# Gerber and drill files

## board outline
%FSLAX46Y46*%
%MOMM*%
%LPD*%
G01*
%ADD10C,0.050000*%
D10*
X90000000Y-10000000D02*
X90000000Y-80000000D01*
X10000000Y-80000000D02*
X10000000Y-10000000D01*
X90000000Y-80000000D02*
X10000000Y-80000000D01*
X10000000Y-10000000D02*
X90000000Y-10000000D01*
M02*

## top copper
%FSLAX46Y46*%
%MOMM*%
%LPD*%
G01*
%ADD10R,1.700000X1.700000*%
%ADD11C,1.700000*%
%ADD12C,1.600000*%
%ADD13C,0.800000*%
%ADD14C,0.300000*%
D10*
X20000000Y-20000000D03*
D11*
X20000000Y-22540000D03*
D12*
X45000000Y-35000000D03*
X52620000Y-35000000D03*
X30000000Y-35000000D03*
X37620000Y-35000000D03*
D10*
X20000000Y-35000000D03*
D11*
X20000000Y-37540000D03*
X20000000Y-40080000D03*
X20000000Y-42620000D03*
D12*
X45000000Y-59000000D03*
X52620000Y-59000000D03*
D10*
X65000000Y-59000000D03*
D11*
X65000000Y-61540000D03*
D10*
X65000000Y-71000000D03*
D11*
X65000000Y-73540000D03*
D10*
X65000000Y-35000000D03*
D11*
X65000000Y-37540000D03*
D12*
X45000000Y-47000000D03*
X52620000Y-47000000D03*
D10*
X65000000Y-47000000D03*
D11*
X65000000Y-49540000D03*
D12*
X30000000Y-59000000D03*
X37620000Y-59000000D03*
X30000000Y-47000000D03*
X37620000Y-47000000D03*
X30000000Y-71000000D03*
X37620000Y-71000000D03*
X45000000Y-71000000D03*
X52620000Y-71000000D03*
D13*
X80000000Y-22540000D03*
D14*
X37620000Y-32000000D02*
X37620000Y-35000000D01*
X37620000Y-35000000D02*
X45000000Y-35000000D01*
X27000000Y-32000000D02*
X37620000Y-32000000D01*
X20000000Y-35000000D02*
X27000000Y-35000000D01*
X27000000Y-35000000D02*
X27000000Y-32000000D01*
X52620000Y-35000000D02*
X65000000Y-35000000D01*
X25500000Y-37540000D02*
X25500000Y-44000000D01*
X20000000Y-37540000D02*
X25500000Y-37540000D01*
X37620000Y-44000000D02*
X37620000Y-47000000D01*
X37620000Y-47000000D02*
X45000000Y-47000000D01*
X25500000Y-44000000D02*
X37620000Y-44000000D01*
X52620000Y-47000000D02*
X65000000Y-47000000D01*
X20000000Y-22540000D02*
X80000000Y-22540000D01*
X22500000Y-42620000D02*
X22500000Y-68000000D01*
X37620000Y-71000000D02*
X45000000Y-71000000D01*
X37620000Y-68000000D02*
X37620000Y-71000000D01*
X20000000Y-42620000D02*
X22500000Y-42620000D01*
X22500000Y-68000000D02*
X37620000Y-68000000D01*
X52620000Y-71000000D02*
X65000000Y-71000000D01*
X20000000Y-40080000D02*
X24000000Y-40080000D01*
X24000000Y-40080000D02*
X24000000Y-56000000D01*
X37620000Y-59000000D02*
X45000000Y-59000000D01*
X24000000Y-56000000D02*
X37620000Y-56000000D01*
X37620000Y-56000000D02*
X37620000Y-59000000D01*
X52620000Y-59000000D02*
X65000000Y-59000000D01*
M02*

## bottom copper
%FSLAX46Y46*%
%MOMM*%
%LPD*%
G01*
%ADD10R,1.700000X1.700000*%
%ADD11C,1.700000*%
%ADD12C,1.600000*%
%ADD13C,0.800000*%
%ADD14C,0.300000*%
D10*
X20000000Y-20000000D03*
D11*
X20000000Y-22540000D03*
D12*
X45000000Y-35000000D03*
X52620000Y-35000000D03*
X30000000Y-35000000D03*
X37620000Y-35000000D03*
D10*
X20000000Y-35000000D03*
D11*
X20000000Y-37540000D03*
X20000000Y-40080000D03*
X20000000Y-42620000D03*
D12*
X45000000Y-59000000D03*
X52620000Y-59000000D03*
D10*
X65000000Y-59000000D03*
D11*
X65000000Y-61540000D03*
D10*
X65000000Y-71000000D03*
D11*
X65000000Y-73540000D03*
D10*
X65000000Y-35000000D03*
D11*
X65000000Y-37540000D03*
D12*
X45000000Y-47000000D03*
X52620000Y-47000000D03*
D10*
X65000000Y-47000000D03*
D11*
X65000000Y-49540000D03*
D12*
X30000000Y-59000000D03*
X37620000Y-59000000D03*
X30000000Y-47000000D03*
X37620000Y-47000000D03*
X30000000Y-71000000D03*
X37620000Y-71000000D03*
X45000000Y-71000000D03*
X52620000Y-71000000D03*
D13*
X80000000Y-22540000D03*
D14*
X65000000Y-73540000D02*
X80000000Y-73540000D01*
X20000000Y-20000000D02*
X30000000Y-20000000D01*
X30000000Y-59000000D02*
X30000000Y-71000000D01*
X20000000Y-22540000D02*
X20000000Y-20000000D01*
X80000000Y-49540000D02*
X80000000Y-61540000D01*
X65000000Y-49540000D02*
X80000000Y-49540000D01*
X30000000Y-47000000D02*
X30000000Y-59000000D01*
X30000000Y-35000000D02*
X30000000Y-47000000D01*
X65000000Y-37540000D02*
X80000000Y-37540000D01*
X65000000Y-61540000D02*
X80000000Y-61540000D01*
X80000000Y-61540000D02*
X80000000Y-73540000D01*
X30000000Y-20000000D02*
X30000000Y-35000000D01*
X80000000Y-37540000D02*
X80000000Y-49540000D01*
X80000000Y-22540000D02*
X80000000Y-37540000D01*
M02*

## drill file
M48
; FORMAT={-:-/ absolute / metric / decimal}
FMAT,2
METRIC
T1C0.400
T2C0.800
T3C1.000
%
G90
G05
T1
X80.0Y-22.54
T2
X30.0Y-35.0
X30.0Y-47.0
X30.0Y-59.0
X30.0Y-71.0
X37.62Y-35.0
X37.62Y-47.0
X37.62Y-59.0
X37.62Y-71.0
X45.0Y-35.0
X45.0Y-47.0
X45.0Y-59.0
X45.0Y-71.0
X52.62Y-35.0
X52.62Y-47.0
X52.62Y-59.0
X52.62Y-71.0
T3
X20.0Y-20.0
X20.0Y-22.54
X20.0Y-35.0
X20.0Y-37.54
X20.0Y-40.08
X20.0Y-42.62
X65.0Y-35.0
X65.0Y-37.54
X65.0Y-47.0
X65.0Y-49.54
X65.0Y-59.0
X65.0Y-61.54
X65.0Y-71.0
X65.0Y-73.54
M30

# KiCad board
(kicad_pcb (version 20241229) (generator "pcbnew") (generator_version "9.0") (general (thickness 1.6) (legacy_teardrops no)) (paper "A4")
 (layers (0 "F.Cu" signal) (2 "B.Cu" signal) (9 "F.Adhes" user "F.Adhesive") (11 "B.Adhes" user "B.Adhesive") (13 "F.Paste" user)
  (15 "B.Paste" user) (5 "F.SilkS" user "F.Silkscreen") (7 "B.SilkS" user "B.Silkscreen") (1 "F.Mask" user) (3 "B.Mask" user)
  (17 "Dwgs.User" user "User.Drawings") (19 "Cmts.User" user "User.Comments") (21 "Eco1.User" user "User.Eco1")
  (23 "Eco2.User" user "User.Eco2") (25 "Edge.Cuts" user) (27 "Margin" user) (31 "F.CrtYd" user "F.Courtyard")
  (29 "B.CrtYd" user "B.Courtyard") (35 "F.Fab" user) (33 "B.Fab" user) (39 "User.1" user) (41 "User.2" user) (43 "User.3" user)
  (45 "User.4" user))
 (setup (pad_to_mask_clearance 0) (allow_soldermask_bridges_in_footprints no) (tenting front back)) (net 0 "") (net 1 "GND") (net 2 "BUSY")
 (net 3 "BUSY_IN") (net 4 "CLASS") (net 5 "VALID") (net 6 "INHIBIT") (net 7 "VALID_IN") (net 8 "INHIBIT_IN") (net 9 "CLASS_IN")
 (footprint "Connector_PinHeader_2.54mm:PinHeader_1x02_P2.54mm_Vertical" (layer "F.Cu") (at 20 20)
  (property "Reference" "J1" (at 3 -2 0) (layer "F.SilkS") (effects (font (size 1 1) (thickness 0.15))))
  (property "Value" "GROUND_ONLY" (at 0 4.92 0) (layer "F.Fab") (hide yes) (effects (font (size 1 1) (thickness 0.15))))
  (pad "1" thru_hole rect (at 0 0) (size 1.7 1.7) (drill 1) (layers "*.Cu" "*.Mask") (remove_unused_layers no) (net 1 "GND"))
  (pad "2" thru_hole circle (at 0 2.54) (size 1.7 1.7) (drill 1) (layers "*.Cu" "*.Mask") (remove_unused_layers no) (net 1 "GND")))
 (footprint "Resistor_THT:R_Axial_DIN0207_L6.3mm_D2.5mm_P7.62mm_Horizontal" (layer "F.Cu") (at 45 35)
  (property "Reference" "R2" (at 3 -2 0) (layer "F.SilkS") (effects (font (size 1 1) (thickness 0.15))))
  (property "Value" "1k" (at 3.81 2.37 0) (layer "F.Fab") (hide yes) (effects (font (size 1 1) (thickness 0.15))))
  (pad "1" thru_hole circle (at 0 0) (size 1.6 1.6) (drill 0.8) (layers "*.Cu" "*.Mask") (remove_unused_layers no) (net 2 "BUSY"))
  (pad "2" thru_hole circle (at 7.62 0) (size 1.6 1.6) (drill 0.8) (layers "*.Cu" "*.Mask") (remove_unused_layers no) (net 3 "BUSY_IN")))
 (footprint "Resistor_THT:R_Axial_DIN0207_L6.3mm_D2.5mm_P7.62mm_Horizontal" (layer "F.Cu") (at 30 35)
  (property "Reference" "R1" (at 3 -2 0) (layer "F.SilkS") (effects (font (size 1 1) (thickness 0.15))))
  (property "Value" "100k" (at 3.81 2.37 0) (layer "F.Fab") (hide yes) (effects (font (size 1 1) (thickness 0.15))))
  (pad "1" thru_hole circle (at 0 0) (size 1.6 1.6) (drill 0.8) (layers "*.Cu" "*.Mask") (remove_unused_layers no) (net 1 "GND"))
  (pad "2" thru_hole circle (at 7.62 0) (size 1.6 1.6) (drill 0.8) (layers "*.Cu" "*.Mask") (remove_unused_layers no) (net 2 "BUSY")))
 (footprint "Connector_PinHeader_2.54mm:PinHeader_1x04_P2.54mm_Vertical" (layer "F.Cu") (at 20 35)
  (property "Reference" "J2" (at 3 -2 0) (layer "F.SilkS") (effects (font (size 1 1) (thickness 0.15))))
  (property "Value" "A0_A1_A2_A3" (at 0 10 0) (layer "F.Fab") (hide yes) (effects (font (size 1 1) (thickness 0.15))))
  (pad "1" thru_hole rect (at 0 0) (size 1.7 1.7) (drill 1) (layers "*.Cu" "*.Mask") (remove_unused_layers no) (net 2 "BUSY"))
  (pad "2" thru_hole circle (at 0 2.54) (size 1.7 1.7) (drill 1) (layers "*.Cu" "*.Mask") (remove_unused_layers no) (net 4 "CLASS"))
  (pad "3" thru_hole circle (at 0 5.08) (size 1.7 1.7) (drill 1) (layers "*.Cu" "*.Mask") (remove_unused_layers no) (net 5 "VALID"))
  (pad "4" thru_hole circle (at 0 7.62) (size 1.7 1.7) (drill 1) (layers "*.Cu" "*.Mask") (remove_unused_layers no) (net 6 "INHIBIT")))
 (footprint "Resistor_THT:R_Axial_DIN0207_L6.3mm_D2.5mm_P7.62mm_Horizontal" (layer "F.Cu") (at 45 59)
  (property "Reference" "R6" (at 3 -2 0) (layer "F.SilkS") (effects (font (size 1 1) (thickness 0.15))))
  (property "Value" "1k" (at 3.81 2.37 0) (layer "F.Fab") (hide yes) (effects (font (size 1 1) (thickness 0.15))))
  (pad "1" thru_hole circle (at 0 0) (size 1.6 1.6) (drill 0.8) (layers "*.Cu" "*.Mask") (remove_unused_layers no) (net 5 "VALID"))
  (pad "2" thru_hole circle (at 7.62 0) (size 1.6 1.6) (drill 0.8) (layers "*.Cu" "*.Mask") (remove_unused_layers no) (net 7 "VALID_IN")))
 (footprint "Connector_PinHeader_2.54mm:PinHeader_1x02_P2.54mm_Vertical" (layer "F.Cu") (at 65 59)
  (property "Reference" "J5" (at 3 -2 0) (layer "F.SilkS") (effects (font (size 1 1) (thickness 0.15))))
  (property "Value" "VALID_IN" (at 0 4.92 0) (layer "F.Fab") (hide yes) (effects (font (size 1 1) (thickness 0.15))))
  (pad "1" thru_hole rect (at 0 0) (size 1.7 1.7) (drill 1) (layers "*.Cu" "*.Mask") (remove_unused_layers no) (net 7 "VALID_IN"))
  (pad "2" thru_hole circle (at 0 2.54) (size 1.7 1.7) (drill 1) (layers "*.Cu" "*.Mask") (remove_unused_layers no) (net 1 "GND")))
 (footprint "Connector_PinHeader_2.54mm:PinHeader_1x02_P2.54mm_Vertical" (layer "F.Cu") (at 65 71)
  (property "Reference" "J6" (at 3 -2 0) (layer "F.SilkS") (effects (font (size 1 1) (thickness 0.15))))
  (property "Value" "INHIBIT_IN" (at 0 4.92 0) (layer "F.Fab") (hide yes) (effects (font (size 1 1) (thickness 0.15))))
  (pad "1" thru_hole rect (at 0 0) (size 1.7 1.7) (drill 1) (layers "*.Cu" "*.Mask") (remove_unused_layers no) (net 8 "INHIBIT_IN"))
  (pad "2" thru_hole circle (at 0 2.54) (size 1.7 1.7) (drill 1) (layers "*.Cu" "*.Mask") (remove_unused_layers no) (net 1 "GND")))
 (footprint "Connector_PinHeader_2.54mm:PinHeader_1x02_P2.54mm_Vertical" (layer "F.Cu") (at 65 35)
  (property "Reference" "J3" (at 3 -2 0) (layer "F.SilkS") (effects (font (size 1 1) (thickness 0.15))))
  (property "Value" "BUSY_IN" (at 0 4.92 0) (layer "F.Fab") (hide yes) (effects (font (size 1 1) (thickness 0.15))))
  (pad "1" thru_hole rect (at 0 0) (size 1.7 1.7) (drill 1) (layers "*.Cu" "*.Mask") (remove_unused_layers no) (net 3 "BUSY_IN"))
  (pad "2" thru_hole circle (at 0 2.54) (size 1.7 1.7) (drill 1) (layers "*.Cu" "*.Mask") (remove_unused_layers no) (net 1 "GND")))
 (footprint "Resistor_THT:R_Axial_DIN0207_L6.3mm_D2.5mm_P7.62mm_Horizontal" (layer "F.Cu") (at 45 47)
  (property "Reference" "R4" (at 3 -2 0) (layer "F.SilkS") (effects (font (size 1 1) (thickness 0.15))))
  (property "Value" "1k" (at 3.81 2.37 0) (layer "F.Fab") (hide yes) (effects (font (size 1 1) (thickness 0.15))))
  (pad "1" thru_hole circle (at 0 0) (size 1.6 1.6) (drill 0.8) (layers "*.Cu" "*.Mask") (remove_unused_layers no) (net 4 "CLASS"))
  (pad "2" thru_hole circle (at 7.62 0) (size 1.6 1.6) (drill 0.8) (layers "*.Cu" "*.Mask") (remove_unused_layers no) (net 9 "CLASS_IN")))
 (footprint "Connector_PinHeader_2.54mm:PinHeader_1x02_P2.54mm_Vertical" (layer "F.Cu") (at 65 47)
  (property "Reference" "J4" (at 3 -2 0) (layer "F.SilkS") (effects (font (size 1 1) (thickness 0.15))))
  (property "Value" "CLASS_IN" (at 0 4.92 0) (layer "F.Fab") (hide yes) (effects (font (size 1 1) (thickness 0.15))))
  (pad "1" thru_hole rect (at 0 0) (size 1.7 1.7) (drill 1) (layers "*.Cu" "*.Mask") (remove_unused_layers no) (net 9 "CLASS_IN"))
  (pad "2" thru_hole circle (at 0 2.54) (size 1.7 1.7) (drill 1) (layers "*.Cu" "*.Mask") (remove_unused_layers no) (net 1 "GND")))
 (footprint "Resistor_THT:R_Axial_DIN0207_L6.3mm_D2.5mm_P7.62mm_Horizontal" (layer "F.Cu") (at 30 59)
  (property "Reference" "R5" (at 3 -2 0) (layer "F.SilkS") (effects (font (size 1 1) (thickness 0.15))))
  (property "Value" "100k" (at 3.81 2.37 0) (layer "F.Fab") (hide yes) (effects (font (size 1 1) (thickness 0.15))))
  (pad "1" thru_hole circle (at 0 0) (size 1.6 1.6) (drill 0.8) (layers "*.Cu" "*.Mask") (remove_unused_layers no) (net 1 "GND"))
  (pad "2" thru_hole circle (at 7.62 0) (size 1.6 1.6) (drill 0.8) (layers "*.Cu" "*.Mask") (remove_unused_layers no) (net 5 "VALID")))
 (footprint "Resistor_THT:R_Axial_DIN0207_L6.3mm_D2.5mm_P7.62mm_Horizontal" (layer "F.Cu") (at 30 47)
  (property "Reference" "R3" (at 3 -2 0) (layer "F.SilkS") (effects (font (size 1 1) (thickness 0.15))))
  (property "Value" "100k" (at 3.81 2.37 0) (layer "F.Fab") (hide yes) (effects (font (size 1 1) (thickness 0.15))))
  (pad "1" thru_hole circle (at 0 0) (size 1.6 1.6) (drill 0.8) (layers "*.Cu" "*.Mask") (remove_unused_layers no) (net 1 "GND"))
  (pad "2" thru_hole circle (at 7.62 0) (size 1.6 1.6) (drill 0.8) (layers "*.Cu" "*.Mask") (remove_unused_layers no) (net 4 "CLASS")))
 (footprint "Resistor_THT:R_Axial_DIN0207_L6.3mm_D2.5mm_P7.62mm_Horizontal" (layer "F.Cu") (at 30 71)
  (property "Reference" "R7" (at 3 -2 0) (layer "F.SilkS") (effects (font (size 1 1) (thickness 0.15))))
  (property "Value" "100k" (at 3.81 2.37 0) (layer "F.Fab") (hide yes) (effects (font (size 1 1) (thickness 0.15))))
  (pad "1" thru_hole circle (at 0 0) (size 1.6 1.6) (drill 0.8) (layers "*.Cu" "*.Mask") (remove_unused_layers no) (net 1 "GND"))
  (pad "2" thru_hole circle (at 7.62 0) (size 1.6 1.6) (drill 0.8) (layers "*.Cu" "*.Mask") (remove_unused_layers no) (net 6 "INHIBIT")))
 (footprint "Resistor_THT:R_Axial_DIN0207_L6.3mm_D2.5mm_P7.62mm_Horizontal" (layer "F.Cu") (at 45 71)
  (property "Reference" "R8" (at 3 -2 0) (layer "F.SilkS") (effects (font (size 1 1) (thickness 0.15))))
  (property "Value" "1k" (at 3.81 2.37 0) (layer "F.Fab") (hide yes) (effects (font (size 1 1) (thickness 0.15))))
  (pad "1" thru_hole circle (at 0 0) (size 1.6 1.6) (drill 0.8) (layers "*.Cu" "*.Mask") (remove_unused_layers no) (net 6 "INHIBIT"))
  (pad "2" thru_hole circle (at 7.62 0) (size 1.6 1.6) (drill 0.8) (layers "*.Cu" "*.Mask") (remove_unused_layers no) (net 8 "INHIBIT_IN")))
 (gr_line (start 90 10) (end 90 80) (stroke (width 0.05) (type default)) (layer "Edge.Cuts"))
 (gr_line (start 10 80) (end 10 10) (stroke (width 0.05) (type default)) (layer "Edge.Cuts"))
 (gr_line (start 90 80) (end 10 80) (stroke (width 0.05) (type default)) (layer "Edge.Cuts"))
 (gr_line (start 10 10) (end 90 10) (stroke (width 0.05) (type default)) (layer "Edge.Cuts"))
 (segment (start 37.62 32) (end 37.62 35) (width 0.3) (layer "F.Cu") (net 2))
 (segment (start 37.62 35) (end 45 35) (width 0.3) (layer "F.Cu") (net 2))
 (segment (start 27 32) (end 37.62 32) (width 0.3) (layer "F.Cu") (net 2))
 (segment (start 20 35) (end 27 35) (width 0.3) (layer "F.Cu") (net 2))
 (segment (start 27 35) (end 27 32) (width 0.3) (layer "F.Cu") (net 2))
 (segment (start 52.62 35) (end 65 35) (width 0.3) (layer "F.Cu") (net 3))
 (segment (start 25.5 37.54) (end 25.5 44) (width 0.3) (layer "F.Cu") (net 4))
 (segment (start 20 37.54) (end 25.5 37.54) (width 0.3) (layer "F.Cu") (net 4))
 (segment (start 37.62 44) (end 37.62 47) (width 0.3) (layer "F.Cu") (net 4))
 (segment (start 37.62 47) (end 45 47) (width 0.3) (layer "F.Cu") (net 4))
 (segment (start 25.5 44) (end 37.62 44) (width 0.3) (layer "F.Cu") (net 4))
 (segment (start 52.62 47) (end 65 47) (width 0.3) (layer "F.Cu") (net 9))
 (segment (start 20 22.54) (end 80 22.54) (width 0.3) (layer "F.Cu") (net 1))
 (via (at 80 22.54) (size 0.8) (drill 0.4) (layers "F.Cu" "B.Cu") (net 1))
 (segment (start 65 73.54) (end 80 73.54) (width 0.3) (layer "B.Cu") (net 1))
 (segment (start 20 20) (end 30 20) (width 0.3) (layer "B.Cu") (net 1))
 (segment (start 30 59) (end 30 71) (width 0.3) (layer "B.Cu") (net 1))
 (segment (start 20 22.54) (end 20 20) (width 0.3) (layer "B.Cu") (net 1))
 (segment (start 80 49.54) (end 80 61.54) (width 0.3) (layer "B.Cu") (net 1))
 (segment (start 65 49.54) (end 80 49.54) (width 0.3) (layer "B.Cu") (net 1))
 (segment (start 30 47) (end 30 59) (width 0.3) (layer "B.Cu") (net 1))
 (segment (start 30 35) (end 30 47) (width 0.3) (layer "B.Cu") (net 1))
 (segment (start 65 37.54) (end 80 37.54) (width 0.3) (layer "B.Cu") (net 1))
 (segment (start 65 61.54) (end 80 61.54) (width 0.3) (layer "B.Cu") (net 1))
 (segment (start 80 61.54) (end 80 73.54) (width 0.3) (layer "B.Cu") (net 1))
 (segment (start 30 20) (end 30 35) (width 0.3) (layer "B.Cu") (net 1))
 (segment (start 80 37.54) (end 80 49.54) (width 0.3) (layer "B.Cu") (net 1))
 (segment (start 80 22.54) (end 80 37.54) (width 0.3) (layer "B.Cu") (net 1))
 (segment (start 22.5 42.62) (end 22.5 68) (width 0.3) (layer "F.Cu") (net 6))
 (segment (start 37.62 71) (end 45 71) (width 0.3) (layer "F.Cu") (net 6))
 (segment (start 37.62 68) (end 37.62 71) (width 0.3) (layer "F.Cu") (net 6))
 (segment (start 20 42.62) (end 22.5 42.62) (width 0.3) (layer "F.Cu") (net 6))
 (segment (start 22.5 68) (end 37.62 68) (width 0.3) (layer "F.Cu") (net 6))
 (segment (start 52.62 71) (end 65 71) (width 0.3) (layer "F.Cu") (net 8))
 (segment (start 20 40.08) (end 24 40.08) (width 0.3) (layer "F.Cu") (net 5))
 (segment (start 24 40.08) (end 24 56) (width 0.3) (layer "F.Cu") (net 5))
 (segment (start 37.62 59) (end 45 59) (width 0.3) (layer "F.Cu") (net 5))
 (segment (start 24 56) (end 37.62 56) (width 0.3) (layer "F.Cu") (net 5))
 (segment (start 37.62 56) (end 37.62 59) (width 0.3) (layer "F.Cu") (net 5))
 (segment (start 52.62 59) (end 65 59) (width 0.3) (layer "F.Cu") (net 7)))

